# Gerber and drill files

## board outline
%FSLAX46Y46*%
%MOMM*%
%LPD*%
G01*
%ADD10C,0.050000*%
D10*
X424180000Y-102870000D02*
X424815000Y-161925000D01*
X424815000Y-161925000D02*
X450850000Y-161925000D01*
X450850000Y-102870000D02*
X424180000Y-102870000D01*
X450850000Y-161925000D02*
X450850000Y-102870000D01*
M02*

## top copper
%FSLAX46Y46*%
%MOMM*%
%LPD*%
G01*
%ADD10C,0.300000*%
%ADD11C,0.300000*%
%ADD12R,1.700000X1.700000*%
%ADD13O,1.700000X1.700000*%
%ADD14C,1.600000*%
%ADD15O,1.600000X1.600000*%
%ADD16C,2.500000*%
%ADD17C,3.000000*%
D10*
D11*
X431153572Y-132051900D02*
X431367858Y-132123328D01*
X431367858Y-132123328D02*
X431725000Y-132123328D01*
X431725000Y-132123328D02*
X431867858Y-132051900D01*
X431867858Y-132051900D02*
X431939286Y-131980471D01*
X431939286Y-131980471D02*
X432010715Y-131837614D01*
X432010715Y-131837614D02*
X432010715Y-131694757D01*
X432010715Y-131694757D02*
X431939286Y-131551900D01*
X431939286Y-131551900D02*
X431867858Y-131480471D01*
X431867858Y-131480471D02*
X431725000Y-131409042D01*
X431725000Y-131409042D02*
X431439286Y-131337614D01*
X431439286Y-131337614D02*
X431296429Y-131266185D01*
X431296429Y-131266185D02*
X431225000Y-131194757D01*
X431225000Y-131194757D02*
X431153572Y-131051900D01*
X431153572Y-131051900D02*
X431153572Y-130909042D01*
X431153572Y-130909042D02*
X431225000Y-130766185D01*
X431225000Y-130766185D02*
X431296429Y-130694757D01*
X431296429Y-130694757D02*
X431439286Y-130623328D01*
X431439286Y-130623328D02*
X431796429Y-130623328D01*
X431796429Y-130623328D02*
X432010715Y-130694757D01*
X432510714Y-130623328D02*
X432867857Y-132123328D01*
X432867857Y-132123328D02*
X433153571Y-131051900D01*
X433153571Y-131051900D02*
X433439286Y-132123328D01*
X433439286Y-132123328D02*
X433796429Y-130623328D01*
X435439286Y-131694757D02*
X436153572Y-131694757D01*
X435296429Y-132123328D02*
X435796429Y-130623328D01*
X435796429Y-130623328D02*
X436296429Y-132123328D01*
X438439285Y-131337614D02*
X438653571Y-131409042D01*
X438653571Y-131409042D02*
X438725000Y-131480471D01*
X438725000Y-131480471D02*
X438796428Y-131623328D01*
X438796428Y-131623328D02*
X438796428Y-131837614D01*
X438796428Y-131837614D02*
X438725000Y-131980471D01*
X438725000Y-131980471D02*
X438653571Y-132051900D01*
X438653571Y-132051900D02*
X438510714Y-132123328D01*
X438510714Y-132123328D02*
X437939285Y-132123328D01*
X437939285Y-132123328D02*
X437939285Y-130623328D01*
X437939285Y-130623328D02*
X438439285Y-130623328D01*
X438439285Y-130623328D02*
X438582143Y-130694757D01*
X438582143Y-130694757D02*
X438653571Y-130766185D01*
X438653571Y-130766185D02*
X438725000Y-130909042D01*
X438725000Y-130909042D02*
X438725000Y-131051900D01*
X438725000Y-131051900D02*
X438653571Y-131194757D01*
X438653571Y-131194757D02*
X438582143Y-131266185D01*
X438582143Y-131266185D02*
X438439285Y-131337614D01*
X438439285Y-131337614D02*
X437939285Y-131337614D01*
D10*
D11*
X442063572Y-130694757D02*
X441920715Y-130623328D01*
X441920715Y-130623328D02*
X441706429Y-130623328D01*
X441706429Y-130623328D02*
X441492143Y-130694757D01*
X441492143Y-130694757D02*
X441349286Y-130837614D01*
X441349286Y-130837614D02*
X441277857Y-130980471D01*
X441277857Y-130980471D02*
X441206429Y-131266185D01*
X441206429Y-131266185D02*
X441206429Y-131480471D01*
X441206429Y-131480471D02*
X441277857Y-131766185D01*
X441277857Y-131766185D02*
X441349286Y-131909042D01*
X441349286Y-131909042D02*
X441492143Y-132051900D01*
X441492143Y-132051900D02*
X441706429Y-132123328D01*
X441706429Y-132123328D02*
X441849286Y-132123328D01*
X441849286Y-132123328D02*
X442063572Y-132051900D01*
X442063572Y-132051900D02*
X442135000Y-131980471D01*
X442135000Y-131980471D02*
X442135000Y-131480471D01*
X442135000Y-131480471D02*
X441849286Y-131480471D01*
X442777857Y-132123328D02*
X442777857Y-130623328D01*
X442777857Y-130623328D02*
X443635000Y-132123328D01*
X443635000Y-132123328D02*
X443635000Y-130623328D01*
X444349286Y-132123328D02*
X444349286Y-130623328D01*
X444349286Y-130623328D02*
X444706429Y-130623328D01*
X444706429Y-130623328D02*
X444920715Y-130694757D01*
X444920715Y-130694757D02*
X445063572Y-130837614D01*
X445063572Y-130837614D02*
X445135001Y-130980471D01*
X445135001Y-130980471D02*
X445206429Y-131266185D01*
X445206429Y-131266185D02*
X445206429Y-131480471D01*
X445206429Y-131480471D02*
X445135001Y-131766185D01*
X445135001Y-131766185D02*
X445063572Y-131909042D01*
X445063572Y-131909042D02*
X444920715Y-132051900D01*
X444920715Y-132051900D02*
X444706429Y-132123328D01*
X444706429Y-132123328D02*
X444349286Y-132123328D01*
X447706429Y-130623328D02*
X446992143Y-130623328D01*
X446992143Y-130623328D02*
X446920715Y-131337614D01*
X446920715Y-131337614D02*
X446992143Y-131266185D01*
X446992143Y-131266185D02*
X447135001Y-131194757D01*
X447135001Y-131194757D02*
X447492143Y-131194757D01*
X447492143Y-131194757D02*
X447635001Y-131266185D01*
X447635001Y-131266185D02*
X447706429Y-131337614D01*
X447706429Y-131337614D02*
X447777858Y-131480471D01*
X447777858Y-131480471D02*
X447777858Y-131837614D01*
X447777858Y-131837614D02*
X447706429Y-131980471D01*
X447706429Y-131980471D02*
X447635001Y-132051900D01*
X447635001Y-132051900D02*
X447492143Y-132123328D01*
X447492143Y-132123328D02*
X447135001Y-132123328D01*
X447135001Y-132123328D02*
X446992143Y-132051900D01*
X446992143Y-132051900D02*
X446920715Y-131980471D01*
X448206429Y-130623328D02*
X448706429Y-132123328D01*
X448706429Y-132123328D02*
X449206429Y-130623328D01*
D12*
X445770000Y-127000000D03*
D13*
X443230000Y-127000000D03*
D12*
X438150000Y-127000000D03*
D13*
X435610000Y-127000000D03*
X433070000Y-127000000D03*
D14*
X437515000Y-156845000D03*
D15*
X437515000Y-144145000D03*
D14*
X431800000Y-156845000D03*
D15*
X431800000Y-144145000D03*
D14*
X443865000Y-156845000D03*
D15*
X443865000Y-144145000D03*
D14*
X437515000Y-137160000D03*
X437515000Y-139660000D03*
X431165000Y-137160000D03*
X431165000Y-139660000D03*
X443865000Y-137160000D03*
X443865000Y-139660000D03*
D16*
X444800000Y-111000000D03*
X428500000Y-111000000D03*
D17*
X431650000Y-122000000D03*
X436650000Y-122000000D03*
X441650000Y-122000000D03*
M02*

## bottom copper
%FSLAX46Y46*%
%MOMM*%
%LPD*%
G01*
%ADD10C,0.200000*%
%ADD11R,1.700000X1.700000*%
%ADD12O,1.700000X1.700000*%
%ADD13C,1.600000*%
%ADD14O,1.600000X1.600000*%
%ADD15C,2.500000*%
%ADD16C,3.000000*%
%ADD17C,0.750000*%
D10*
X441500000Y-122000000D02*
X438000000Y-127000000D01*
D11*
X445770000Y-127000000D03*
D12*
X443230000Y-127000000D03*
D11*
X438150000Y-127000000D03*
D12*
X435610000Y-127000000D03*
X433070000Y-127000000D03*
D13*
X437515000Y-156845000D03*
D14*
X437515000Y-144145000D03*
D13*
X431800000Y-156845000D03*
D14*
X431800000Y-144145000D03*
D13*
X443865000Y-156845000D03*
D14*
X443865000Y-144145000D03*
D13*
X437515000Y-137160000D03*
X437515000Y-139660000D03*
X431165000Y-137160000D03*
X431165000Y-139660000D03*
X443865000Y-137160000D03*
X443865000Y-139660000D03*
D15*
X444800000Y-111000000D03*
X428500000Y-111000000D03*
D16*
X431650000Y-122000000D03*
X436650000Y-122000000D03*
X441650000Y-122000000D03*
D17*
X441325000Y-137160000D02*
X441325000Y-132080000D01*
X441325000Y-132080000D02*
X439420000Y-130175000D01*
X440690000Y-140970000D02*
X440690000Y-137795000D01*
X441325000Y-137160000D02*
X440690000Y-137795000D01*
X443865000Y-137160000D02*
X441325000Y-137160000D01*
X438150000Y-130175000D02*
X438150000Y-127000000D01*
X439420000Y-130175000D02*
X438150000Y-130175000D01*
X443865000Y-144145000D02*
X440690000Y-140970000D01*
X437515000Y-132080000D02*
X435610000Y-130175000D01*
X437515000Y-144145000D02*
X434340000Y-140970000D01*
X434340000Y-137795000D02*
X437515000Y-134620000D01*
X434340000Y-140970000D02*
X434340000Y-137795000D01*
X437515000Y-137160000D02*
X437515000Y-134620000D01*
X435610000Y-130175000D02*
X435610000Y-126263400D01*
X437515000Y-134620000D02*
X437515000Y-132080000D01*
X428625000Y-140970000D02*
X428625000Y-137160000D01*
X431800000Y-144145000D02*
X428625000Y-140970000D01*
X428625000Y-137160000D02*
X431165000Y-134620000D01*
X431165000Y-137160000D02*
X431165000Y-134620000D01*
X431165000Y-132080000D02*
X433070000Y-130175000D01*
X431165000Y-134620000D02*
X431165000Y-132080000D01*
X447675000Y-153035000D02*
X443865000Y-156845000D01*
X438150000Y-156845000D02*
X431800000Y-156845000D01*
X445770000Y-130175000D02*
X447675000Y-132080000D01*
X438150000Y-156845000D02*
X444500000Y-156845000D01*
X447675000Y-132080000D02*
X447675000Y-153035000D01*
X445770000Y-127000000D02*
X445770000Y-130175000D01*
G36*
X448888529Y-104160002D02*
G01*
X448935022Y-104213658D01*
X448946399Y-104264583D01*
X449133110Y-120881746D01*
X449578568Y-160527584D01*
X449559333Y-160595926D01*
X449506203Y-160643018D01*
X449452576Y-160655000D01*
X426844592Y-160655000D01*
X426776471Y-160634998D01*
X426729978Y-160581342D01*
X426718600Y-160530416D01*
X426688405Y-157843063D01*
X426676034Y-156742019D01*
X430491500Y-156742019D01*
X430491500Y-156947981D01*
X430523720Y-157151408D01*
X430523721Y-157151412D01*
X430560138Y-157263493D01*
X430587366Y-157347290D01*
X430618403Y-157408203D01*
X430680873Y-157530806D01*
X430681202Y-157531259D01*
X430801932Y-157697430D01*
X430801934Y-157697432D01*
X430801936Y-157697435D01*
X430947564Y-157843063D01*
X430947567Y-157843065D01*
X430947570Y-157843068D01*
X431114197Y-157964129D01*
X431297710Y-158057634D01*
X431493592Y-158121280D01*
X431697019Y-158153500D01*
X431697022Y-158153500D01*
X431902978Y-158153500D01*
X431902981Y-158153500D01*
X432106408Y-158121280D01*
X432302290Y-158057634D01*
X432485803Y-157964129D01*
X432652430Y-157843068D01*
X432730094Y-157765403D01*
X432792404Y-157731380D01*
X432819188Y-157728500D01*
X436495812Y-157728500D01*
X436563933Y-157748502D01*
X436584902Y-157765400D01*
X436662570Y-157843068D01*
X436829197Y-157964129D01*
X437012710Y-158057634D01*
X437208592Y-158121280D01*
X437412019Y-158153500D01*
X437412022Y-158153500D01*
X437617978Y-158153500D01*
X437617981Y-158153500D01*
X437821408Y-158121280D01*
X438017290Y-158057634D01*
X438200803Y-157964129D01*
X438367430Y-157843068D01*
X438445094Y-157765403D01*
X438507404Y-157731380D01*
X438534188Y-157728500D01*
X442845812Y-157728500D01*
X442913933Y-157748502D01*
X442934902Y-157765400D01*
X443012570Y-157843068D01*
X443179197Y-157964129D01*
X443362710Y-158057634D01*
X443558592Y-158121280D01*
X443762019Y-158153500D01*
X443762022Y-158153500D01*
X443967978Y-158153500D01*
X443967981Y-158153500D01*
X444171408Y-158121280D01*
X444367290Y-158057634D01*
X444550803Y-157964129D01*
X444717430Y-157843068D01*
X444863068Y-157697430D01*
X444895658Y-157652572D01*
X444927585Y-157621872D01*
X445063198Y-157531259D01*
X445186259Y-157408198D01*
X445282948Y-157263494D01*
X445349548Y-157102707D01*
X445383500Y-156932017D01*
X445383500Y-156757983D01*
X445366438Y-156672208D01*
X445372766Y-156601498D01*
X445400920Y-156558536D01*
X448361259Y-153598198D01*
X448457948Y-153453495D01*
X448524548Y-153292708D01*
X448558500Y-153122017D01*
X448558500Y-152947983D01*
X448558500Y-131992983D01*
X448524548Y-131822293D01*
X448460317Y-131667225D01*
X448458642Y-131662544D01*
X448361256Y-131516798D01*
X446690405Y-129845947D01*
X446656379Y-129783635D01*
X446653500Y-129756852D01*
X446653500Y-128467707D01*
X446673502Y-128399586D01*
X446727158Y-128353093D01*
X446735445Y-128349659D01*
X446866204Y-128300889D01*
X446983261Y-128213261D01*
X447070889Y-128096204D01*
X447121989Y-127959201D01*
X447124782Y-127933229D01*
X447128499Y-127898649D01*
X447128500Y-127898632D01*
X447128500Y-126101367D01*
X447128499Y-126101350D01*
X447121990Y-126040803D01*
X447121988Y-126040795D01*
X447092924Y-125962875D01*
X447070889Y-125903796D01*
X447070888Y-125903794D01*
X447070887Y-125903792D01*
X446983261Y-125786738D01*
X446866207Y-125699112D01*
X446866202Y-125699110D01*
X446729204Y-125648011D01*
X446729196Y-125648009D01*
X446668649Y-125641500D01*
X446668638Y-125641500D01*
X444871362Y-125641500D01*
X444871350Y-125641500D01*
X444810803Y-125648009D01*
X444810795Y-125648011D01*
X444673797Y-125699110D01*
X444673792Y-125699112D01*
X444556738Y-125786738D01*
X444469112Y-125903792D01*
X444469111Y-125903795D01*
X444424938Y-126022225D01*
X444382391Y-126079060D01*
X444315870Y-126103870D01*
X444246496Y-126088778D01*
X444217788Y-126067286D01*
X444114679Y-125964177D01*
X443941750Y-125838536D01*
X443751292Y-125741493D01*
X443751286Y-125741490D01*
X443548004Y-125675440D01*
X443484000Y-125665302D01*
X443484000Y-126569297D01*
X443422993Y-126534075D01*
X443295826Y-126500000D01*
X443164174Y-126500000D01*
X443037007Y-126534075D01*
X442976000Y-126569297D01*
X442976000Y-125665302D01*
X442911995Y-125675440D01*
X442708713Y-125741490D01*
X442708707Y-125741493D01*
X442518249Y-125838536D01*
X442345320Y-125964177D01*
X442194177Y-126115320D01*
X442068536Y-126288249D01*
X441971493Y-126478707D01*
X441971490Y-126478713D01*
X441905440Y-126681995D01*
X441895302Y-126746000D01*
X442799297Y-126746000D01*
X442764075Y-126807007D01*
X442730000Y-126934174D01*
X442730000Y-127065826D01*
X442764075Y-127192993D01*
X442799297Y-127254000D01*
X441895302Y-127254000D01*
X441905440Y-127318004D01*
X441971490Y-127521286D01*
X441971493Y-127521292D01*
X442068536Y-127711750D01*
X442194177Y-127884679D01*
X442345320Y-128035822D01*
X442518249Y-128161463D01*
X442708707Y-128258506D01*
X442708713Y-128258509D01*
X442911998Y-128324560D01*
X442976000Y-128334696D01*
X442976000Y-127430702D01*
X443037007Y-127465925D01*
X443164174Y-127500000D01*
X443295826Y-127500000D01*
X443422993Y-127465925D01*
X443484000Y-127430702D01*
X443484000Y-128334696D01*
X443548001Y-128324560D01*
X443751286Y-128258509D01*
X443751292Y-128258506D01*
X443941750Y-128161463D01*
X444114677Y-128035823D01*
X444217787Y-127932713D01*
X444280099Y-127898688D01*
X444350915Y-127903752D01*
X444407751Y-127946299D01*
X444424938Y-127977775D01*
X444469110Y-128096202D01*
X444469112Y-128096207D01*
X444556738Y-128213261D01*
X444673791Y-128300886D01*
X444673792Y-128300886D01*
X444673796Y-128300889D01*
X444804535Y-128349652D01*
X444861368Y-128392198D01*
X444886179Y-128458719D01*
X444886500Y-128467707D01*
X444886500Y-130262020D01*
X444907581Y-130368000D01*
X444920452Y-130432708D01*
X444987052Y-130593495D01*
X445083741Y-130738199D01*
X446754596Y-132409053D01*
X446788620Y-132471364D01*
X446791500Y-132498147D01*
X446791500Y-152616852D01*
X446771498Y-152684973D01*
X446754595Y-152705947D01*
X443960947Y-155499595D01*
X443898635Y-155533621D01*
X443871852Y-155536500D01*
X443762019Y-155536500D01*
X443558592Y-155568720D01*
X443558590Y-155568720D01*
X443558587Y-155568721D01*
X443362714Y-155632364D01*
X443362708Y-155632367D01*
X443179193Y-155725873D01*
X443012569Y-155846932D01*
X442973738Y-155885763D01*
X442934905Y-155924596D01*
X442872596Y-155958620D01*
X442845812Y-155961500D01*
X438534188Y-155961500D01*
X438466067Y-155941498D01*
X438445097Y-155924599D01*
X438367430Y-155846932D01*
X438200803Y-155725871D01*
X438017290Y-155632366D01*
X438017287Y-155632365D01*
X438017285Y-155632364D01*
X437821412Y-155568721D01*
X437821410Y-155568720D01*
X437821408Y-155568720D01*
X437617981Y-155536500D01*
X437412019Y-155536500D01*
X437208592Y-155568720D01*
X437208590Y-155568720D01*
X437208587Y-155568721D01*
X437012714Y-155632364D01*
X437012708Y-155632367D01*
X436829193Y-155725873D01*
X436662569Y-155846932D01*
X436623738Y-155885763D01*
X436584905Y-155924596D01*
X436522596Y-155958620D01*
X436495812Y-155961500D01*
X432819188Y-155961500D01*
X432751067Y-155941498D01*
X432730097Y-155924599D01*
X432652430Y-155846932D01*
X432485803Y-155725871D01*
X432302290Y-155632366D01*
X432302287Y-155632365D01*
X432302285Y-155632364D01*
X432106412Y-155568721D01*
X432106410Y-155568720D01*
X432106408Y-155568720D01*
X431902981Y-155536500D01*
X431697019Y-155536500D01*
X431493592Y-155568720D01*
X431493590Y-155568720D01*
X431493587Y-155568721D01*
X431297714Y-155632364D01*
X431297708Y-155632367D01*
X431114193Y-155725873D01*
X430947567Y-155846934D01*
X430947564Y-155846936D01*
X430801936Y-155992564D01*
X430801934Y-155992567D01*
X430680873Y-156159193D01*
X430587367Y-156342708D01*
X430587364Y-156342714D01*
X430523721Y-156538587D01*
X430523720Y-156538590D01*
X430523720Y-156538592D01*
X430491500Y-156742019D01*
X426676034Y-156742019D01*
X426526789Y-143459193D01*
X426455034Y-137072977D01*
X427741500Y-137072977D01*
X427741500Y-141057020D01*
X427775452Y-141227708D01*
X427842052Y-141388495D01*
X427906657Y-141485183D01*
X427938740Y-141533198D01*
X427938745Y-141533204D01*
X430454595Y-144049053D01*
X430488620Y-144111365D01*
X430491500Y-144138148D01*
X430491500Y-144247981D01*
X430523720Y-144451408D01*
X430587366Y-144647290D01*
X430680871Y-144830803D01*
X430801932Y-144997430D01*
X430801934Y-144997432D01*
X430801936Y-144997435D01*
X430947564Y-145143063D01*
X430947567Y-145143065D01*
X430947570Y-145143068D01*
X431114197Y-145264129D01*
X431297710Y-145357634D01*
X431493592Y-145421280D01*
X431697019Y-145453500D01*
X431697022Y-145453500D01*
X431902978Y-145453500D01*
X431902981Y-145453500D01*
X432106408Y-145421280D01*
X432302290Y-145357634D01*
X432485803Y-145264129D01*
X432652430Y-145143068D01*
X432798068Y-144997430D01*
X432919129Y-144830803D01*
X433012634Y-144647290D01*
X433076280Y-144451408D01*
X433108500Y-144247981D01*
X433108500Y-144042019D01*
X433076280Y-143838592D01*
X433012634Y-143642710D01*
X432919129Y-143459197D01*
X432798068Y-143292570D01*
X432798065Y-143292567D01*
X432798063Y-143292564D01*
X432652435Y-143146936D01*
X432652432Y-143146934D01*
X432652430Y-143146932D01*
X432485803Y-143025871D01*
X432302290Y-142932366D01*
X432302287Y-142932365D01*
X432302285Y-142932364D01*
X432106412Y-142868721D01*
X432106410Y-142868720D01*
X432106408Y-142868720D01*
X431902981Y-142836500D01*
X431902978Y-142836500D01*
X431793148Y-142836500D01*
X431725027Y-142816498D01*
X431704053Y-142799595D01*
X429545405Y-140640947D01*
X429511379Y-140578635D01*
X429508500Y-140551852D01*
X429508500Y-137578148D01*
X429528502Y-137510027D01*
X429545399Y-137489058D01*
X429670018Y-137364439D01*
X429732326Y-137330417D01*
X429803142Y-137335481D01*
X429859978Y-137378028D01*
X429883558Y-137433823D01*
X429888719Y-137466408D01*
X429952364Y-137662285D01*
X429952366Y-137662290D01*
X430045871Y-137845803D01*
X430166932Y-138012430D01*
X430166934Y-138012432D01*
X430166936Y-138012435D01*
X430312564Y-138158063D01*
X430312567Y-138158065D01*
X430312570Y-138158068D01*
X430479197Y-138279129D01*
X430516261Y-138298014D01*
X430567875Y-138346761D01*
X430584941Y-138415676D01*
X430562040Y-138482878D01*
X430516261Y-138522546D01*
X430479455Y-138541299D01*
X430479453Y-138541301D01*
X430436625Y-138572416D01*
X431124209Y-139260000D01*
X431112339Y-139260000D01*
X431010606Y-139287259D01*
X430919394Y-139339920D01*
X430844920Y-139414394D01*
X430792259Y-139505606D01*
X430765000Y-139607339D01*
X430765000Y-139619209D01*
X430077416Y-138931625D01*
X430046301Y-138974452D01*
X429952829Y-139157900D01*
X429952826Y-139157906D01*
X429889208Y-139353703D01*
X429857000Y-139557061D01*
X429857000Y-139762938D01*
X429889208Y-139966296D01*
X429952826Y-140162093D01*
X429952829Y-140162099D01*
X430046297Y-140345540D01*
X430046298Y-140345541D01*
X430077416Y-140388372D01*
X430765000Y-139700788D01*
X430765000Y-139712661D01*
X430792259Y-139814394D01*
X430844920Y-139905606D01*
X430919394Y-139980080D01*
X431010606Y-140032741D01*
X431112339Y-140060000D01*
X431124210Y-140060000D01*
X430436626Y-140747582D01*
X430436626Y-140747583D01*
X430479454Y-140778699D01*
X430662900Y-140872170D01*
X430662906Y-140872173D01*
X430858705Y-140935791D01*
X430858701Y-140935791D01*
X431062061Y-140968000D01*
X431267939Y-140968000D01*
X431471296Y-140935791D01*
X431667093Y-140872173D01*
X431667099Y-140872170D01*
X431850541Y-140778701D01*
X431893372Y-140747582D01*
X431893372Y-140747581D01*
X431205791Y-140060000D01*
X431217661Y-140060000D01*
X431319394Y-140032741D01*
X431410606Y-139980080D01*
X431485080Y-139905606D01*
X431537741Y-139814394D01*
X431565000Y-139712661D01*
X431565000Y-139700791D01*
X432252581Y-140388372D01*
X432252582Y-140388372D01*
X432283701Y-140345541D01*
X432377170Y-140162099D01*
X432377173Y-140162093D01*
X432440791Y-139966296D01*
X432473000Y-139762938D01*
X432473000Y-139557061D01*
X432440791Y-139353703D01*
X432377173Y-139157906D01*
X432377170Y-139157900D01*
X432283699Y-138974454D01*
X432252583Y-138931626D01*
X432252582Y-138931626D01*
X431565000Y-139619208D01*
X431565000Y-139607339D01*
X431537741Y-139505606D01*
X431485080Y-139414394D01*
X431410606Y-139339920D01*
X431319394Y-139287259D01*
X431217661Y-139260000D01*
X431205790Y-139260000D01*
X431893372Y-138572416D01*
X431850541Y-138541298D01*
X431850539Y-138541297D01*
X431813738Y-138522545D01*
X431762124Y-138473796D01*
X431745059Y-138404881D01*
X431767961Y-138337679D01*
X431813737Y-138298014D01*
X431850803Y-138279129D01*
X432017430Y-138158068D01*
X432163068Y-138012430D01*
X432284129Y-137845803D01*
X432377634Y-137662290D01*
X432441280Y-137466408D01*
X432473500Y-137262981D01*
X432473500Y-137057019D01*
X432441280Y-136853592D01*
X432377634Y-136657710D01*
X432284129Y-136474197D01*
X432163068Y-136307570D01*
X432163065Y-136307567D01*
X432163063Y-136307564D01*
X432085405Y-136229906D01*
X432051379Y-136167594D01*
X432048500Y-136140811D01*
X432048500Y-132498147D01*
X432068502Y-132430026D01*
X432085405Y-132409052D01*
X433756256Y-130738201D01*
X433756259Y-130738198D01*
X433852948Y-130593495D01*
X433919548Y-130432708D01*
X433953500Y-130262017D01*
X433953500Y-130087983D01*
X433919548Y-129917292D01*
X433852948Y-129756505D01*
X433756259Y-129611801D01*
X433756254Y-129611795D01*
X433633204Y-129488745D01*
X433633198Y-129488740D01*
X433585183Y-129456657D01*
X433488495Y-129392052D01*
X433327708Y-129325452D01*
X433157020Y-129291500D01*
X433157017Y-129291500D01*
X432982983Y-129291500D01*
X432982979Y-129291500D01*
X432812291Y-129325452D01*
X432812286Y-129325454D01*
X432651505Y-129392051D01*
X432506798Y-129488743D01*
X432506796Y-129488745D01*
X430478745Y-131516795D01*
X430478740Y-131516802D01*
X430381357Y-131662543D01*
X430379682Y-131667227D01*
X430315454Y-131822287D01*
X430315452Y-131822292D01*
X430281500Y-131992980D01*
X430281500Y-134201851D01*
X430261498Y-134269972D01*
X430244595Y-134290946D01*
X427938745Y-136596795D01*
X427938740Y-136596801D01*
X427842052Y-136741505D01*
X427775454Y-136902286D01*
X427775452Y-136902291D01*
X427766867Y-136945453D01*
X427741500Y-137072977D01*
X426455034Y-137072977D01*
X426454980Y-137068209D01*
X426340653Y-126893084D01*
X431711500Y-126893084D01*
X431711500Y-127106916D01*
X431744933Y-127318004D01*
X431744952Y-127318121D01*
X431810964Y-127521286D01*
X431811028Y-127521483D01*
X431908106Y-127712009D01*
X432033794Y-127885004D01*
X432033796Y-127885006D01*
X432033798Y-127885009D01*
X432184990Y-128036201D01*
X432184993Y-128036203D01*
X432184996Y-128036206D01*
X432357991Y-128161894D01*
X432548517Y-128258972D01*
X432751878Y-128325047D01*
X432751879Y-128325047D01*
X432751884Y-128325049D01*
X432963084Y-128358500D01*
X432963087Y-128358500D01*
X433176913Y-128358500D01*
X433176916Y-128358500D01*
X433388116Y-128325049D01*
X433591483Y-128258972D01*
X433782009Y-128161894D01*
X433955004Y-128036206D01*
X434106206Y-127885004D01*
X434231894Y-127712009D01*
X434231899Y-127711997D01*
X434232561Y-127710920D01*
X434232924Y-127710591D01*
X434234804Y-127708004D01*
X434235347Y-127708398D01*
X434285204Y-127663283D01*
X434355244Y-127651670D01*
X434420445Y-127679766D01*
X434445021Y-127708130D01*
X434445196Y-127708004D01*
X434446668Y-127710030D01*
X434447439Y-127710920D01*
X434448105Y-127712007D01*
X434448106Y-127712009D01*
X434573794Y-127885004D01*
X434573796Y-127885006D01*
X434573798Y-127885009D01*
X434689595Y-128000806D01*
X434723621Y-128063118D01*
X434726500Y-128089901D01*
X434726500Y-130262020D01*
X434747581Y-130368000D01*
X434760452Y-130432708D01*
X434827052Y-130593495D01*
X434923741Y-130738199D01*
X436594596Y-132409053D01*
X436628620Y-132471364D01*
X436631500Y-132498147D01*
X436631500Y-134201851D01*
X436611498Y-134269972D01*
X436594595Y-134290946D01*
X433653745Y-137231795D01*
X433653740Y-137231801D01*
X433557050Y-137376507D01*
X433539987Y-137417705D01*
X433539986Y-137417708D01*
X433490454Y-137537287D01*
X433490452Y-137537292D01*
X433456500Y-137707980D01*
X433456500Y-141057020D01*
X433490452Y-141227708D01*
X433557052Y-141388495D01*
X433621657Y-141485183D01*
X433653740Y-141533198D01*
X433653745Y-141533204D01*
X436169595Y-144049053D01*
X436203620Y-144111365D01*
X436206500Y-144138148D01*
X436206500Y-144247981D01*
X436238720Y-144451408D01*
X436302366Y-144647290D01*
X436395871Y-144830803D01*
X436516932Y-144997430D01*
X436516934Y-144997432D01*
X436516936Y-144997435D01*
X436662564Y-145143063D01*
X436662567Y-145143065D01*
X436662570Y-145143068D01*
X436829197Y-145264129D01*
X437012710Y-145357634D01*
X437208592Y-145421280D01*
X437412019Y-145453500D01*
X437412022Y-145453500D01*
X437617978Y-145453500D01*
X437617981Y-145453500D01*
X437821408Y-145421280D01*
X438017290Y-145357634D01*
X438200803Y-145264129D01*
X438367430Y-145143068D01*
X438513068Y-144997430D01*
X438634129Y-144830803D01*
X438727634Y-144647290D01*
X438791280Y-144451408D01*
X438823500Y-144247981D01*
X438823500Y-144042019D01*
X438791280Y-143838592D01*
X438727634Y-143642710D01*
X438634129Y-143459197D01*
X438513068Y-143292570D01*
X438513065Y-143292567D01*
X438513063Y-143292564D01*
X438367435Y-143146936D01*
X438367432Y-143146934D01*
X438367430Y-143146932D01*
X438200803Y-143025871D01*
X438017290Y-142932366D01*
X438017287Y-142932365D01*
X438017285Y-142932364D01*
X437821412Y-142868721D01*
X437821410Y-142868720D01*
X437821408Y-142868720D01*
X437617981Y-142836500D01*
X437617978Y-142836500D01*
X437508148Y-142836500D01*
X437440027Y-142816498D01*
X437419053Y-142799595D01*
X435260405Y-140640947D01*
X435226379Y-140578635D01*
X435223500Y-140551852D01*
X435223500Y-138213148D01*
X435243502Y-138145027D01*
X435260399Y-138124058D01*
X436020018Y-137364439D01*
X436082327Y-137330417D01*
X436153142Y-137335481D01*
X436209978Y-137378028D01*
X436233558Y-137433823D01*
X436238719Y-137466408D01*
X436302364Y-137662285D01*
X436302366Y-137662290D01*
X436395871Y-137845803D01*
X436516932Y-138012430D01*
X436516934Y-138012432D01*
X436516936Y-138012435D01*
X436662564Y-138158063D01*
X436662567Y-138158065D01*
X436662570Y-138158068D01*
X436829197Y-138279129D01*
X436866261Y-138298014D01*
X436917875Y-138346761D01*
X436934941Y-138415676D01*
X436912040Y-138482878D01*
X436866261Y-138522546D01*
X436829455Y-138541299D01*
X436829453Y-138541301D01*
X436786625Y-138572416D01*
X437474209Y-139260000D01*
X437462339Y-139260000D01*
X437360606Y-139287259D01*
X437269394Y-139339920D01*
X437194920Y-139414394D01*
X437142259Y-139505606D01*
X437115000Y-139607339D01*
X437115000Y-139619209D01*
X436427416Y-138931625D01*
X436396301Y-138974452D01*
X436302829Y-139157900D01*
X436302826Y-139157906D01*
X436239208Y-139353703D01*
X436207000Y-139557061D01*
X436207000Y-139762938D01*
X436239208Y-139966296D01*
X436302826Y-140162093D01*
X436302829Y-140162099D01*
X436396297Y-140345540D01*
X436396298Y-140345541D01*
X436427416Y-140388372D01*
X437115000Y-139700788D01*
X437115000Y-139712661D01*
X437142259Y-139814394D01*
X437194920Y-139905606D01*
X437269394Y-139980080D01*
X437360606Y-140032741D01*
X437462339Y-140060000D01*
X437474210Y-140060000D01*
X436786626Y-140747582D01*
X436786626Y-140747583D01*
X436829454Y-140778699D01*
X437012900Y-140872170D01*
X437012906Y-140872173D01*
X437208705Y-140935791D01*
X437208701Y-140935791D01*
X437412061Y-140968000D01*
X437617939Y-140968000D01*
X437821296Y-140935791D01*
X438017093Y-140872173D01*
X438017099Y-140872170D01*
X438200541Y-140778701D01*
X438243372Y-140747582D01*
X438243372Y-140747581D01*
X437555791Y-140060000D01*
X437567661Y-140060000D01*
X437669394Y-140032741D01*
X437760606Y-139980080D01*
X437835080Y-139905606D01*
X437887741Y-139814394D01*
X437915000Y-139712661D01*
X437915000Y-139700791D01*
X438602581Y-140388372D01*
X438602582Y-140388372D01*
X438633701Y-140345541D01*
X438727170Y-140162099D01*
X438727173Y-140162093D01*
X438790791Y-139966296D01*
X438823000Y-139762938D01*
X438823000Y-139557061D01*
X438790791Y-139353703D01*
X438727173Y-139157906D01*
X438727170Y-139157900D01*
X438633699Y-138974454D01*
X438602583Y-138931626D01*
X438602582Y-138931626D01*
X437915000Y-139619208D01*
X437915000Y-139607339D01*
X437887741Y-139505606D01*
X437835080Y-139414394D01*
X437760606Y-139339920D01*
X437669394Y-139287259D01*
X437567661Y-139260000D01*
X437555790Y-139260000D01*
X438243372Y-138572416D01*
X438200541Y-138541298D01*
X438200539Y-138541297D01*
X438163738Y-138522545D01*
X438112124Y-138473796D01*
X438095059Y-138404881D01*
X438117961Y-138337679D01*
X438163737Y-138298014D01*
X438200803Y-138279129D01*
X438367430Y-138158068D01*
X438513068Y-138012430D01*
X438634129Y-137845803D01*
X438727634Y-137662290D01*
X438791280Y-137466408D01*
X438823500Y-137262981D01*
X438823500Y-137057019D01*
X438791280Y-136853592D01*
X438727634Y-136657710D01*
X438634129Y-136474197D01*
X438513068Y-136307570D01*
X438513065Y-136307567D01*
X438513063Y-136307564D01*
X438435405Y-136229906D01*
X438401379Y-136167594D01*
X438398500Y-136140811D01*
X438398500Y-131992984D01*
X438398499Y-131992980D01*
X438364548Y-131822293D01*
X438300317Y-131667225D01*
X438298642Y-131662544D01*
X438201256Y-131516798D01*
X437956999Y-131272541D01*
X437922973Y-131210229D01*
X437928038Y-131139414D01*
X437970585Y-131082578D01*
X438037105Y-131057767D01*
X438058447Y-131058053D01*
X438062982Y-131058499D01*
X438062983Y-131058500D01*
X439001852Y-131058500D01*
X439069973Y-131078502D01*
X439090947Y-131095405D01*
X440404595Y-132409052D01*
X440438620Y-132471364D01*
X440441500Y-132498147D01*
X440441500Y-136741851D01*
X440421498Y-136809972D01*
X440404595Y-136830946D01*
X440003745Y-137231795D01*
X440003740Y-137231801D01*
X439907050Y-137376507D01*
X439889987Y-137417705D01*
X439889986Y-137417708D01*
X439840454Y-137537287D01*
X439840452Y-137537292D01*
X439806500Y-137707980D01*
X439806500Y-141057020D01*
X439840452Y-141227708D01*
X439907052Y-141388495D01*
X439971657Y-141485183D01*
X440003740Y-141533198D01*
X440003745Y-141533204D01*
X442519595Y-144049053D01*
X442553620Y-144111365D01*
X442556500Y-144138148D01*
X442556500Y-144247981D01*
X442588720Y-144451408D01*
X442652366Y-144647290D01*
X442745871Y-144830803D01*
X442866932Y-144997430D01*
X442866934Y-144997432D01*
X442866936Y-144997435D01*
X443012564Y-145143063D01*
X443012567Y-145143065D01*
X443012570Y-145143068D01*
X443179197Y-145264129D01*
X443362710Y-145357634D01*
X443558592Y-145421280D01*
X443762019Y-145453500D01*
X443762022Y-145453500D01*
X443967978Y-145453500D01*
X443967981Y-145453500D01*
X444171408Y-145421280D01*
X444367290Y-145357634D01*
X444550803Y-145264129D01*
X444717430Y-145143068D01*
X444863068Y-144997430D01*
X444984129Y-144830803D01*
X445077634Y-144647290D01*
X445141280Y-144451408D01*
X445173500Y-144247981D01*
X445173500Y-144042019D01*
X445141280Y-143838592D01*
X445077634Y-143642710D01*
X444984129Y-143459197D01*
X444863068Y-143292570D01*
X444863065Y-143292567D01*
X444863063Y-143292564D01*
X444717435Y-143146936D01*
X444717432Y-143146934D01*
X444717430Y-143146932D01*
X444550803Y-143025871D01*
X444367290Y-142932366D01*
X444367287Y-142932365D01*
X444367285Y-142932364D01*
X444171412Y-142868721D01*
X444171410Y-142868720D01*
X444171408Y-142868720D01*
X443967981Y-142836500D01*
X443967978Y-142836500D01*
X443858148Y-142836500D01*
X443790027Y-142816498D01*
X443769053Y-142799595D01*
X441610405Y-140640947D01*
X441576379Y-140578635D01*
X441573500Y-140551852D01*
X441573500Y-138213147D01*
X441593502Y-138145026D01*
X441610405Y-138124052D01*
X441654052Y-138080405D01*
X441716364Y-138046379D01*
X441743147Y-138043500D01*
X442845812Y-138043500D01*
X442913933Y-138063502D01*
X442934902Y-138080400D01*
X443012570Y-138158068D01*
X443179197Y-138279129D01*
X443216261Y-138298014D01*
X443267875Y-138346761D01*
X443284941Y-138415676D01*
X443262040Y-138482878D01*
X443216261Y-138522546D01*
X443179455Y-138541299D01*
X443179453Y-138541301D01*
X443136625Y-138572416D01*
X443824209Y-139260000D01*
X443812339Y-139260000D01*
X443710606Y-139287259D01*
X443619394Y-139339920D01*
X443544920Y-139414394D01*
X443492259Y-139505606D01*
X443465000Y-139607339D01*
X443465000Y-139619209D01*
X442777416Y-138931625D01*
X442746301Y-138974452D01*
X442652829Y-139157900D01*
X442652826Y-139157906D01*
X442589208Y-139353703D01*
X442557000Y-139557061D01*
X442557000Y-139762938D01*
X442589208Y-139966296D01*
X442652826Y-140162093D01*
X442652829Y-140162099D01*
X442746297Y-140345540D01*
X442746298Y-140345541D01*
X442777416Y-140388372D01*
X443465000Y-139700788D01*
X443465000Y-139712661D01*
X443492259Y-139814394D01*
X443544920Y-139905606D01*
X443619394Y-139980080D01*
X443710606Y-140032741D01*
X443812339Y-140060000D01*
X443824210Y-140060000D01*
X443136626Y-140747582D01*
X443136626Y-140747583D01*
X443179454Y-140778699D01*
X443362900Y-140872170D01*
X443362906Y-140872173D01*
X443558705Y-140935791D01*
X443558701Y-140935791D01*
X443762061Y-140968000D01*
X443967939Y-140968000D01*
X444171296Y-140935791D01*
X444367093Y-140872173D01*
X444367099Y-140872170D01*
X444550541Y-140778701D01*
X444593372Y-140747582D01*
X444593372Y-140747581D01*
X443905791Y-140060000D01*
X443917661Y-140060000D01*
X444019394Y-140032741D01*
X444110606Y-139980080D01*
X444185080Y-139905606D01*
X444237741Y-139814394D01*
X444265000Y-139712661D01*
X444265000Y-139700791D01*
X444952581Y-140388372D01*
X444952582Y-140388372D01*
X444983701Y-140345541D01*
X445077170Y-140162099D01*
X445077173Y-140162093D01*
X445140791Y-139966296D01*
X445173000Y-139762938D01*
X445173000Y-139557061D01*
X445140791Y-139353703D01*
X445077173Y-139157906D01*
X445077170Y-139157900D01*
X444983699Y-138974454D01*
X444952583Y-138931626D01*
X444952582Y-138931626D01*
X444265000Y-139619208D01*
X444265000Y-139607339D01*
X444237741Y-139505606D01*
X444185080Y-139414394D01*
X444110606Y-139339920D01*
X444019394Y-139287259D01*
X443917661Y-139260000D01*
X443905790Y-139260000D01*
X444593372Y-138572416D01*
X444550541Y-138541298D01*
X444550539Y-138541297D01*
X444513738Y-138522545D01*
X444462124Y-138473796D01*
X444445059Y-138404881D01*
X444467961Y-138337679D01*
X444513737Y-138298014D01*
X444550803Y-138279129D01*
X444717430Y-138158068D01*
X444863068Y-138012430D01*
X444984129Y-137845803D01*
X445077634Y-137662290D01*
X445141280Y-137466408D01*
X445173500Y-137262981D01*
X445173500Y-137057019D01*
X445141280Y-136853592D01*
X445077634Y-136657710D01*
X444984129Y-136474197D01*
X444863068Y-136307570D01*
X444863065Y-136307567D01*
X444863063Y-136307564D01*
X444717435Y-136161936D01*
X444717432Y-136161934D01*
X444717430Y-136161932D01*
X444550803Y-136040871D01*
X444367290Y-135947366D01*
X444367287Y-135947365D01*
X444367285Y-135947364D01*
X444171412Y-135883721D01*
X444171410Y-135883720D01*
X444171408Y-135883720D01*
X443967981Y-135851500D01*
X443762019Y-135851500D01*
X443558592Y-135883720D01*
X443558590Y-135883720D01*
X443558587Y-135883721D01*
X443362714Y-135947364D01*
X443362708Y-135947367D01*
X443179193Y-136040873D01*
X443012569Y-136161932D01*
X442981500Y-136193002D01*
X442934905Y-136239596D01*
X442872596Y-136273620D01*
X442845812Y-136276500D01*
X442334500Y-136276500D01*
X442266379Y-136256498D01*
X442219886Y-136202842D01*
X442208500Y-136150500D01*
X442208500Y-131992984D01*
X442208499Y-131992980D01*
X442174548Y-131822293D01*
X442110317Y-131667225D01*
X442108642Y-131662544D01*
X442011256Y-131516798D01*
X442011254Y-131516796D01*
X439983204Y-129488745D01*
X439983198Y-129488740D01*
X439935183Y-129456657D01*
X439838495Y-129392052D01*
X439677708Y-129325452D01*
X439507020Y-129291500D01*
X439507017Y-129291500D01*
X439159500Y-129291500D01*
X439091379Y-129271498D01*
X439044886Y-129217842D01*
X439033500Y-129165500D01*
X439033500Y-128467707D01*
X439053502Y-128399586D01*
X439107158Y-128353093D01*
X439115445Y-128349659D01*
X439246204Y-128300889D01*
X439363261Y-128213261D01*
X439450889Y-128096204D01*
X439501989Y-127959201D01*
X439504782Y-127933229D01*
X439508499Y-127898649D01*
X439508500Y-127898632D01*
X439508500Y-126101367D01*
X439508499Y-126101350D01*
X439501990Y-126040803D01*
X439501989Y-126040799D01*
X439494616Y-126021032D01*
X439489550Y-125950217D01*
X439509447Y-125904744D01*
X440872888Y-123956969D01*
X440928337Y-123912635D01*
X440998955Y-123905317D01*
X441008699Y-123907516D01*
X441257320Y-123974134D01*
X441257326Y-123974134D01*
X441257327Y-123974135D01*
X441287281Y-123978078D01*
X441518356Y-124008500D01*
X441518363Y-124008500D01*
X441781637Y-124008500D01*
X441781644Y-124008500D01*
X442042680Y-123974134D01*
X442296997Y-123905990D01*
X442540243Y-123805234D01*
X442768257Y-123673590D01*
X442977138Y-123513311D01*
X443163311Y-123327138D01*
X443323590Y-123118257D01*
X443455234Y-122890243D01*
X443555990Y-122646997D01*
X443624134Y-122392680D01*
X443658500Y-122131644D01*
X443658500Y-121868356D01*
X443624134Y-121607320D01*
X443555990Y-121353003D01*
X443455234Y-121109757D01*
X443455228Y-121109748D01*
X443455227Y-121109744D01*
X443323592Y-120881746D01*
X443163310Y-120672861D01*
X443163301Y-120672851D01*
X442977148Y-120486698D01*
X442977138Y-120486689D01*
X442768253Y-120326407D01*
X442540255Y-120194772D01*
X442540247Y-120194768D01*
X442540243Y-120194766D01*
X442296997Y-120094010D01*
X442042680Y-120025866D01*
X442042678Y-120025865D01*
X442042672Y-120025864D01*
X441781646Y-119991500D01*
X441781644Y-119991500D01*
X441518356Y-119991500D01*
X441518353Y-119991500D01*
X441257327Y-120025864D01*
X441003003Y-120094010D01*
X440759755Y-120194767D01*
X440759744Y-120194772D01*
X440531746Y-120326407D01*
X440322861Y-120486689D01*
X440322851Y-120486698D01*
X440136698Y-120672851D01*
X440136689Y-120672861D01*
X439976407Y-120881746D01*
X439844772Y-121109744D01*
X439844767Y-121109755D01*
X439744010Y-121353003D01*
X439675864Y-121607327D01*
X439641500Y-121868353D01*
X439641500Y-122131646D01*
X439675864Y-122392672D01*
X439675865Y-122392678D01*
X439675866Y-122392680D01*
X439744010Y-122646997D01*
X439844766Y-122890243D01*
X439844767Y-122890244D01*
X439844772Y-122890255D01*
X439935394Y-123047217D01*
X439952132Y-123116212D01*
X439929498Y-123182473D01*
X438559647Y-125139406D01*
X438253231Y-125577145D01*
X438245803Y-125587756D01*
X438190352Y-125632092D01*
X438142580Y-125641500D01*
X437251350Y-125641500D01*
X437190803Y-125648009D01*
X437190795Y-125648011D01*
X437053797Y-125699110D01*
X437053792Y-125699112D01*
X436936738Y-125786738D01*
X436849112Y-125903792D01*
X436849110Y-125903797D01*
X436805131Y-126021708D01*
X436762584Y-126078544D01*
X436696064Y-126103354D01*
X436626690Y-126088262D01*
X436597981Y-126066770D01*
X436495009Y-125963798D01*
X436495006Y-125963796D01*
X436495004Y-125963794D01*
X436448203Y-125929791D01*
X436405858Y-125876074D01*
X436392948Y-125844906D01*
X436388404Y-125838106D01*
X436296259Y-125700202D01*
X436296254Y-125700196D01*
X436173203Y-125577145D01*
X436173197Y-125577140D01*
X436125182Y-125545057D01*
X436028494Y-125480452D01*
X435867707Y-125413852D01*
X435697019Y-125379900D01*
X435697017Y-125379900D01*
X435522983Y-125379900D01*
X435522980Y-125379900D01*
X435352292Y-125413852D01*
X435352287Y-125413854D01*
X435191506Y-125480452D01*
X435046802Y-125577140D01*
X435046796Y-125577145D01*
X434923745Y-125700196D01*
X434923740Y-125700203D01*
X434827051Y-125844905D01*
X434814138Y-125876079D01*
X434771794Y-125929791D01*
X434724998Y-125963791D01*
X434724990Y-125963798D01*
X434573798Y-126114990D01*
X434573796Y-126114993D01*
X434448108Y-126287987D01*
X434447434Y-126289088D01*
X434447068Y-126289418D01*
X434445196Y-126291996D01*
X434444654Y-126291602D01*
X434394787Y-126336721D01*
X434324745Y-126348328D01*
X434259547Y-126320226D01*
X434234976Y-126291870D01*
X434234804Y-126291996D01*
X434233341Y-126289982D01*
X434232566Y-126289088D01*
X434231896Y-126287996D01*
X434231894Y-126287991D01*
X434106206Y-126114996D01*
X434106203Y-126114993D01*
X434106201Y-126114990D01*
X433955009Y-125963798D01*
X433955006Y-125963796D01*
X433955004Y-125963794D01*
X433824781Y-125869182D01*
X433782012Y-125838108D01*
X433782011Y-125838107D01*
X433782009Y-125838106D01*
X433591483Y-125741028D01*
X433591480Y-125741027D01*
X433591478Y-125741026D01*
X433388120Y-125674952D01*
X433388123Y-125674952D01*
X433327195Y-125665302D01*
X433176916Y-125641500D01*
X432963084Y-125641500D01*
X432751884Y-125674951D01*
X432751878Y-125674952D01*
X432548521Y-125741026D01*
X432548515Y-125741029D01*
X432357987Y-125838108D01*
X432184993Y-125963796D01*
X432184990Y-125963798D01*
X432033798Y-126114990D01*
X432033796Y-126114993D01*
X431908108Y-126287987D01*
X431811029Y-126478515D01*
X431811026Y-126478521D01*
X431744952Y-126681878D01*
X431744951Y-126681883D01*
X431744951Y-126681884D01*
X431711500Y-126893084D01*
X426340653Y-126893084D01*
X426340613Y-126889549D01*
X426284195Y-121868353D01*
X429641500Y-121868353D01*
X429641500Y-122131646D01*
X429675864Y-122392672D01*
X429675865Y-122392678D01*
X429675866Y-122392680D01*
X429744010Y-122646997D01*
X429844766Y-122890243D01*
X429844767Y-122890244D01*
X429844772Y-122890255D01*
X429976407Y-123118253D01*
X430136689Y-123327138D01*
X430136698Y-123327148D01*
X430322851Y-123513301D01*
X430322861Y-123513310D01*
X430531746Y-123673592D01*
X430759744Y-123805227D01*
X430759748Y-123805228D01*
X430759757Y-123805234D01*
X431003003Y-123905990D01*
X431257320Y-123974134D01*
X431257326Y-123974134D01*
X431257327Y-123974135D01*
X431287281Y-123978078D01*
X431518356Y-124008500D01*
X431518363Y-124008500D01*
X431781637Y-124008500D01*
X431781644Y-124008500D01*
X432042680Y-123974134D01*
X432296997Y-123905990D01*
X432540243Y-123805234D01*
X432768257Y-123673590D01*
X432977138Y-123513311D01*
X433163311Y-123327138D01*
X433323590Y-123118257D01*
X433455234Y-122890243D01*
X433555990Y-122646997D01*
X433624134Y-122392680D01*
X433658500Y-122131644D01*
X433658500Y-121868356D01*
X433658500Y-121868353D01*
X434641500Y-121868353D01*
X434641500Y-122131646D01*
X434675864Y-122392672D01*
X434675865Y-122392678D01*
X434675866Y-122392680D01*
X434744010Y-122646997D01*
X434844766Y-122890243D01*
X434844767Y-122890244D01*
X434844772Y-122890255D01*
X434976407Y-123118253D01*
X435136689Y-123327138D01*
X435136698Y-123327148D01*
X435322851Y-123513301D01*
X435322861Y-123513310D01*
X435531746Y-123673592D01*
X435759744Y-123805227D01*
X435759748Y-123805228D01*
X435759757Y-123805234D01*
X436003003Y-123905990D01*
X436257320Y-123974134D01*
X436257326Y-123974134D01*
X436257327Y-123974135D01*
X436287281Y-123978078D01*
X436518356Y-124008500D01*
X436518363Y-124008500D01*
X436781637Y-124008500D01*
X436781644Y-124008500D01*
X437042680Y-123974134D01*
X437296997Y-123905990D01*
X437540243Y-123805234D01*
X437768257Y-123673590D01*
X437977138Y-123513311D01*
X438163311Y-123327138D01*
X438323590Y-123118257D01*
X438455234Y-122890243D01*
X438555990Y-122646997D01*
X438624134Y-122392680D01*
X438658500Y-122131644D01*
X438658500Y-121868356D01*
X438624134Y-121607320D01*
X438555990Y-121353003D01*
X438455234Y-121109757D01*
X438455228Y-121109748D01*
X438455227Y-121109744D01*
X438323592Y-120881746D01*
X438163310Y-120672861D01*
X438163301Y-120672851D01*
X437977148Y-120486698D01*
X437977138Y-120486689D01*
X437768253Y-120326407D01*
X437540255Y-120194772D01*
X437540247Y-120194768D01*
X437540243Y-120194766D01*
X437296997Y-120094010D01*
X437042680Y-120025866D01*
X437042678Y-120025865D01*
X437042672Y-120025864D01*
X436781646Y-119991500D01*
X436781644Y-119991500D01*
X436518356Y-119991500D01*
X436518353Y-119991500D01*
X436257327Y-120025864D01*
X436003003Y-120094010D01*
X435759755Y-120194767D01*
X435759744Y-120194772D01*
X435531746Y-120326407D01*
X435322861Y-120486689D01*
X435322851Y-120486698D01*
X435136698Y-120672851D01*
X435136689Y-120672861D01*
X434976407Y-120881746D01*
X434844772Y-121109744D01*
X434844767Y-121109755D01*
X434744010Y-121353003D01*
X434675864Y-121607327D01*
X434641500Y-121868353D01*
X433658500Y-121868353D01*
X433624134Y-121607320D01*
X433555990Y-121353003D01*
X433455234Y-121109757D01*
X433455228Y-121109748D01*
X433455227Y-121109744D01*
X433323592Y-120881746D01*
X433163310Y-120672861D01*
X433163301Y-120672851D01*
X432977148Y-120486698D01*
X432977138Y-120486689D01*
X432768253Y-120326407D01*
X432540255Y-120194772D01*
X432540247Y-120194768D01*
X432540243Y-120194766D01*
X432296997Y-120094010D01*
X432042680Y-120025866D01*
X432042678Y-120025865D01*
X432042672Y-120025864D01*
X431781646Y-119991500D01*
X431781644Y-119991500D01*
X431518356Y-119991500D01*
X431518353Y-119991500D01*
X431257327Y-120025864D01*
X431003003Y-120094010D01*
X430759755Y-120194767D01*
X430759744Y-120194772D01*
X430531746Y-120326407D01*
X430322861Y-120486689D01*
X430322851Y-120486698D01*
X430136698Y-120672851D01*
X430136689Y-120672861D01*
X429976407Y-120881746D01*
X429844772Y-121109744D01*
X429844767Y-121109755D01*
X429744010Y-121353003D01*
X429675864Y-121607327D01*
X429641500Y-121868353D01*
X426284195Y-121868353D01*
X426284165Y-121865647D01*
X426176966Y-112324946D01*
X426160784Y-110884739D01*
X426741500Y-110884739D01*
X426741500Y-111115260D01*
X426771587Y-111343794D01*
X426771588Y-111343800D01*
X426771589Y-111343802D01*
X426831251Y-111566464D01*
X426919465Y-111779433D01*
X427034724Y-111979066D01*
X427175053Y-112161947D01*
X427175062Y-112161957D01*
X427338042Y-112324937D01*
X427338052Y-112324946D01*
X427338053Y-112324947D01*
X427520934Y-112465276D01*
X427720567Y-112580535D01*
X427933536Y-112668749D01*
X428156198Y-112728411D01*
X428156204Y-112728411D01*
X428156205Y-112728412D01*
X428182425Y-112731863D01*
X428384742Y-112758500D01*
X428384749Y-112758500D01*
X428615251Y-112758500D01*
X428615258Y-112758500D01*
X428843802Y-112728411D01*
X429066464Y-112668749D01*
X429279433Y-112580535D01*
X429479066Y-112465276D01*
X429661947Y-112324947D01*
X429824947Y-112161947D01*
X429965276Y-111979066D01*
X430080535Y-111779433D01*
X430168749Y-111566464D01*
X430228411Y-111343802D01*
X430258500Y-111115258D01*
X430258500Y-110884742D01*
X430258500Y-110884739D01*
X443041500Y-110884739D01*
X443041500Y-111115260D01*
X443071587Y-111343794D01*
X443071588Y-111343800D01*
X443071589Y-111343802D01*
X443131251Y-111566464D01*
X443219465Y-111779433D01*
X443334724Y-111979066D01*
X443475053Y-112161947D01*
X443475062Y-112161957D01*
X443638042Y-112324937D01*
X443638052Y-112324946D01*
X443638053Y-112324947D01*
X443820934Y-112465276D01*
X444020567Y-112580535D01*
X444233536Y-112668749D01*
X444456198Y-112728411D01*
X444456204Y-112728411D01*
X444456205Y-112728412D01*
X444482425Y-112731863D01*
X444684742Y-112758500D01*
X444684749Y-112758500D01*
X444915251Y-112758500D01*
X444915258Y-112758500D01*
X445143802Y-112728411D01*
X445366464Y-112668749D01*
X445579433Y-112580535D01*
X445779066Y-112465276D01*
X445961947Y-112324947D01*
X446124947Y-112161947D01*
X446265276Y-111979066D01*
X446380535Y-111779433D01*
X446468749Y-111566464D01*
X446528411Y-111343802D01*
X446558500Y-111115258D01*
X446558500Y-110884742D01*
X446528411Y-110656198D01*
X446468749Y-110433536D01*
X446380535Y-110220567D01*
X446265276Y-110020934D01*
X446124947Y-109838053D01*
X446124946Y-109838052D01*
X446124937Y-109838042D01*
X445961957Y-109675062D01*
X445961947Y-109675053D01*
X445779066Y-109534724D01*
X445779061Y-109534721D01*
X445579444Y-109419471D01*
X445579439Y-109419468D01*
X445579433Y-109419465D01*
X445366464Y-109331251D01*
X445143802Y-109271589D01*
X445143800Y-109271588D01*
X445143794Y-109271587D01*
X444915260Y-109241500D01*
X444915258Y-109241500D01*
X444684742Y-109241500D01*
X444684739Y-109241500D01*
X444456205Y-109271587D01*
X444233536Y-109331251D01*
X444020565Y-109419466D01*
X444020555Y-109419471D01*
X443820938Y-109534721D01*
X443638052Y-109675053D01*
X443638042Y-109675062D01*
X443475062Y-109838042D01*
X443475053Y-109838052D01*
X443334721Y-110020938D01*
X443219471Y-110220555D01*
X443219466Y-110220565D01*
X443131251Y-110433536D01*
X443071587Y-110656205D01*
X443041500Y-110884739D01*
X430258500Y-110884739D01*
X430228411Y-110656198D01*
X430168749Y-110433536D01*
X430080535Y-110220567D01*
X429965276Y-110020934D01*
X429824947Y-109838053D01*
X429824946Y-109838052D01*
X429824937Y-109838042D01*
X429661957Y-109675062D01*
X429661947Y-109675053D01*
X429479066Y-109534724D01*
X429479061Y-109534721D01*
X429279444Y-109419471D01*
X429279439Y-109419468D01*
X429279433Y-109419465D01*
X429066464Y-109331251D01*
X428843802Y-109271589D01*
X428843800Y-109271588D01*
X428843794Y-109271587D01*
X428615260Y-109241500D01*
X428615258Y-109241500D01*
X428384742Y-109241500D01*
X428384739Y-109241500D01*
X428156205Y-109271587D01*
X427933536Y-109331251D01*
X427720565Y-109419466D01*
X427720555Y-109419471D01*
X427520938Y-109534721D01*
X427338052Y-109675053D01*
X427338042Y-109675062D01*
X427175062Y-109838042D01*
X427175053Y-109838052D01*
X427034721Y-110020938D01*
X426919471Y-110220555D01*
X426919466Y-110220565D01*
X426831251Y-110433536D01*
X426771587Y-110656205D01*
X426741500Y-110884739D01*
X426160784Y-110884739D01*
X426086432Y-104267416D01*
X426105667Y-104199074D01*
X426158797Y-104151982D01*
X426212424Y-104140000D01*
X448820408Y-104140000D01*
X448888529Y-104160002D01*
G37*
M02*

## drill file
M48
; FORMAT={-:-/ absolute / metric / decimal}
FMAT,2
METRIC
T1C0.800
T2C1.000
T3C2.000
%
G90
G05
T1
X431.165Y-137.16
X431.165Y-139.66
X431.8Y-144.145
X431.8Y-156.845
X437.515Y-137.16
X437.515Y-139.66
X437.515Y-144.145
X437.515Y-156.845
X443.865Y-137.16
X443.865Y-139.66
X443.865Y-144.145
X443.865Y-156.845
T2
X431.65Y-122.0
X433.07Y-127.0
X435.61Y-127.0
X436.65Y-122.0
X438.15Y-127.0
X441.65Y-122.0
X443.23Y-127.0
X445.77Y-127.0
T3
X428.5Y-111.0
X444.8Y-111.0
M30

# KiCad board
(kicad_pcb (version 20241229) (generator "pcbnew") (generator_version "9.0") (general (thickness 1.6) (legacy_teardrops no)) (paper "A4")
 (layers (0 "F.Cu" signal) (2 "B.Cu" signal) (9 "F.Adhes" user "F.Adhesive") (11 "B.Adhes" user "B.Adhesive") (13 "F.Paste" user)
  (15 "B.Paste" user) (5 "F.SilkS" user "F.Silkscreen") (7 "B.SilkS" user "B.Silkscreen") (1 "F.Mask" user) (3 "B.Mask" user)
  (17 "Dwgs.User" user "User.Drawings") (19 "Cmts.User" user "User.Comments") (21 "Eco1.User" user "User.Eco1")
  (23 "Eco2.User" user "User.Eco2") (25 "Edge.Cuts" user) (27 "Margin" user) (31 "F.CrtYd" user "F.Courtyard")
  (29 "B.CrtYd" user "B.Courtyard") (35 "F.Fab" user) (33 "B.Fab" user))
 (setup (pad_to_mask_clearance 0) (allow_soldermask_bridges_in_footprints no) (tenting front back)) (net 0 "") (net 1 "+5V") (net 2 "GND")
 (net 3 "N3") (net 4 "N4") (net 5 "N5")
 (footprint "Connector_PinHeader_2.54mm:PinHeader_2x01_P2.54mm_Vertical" (layer "F.Cu") (at 445.77 127 180)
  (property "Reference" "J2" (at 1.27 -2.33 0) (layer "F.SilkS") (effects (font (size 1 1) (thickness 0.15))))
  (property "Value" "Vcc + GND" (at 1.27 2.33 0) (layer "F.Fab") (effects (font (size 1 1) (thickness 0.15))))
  (pad "1" thru_hole rect (at 0 0 180) (size 1.7 1.7) (drill 1) (layers "*.Cu" "*.Mask") (remove_unused_layers no) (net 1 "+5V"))
  (pad "2" thru_hole oval (at 2.54 0 180) (size 1.7 1.7) (drill 1) (layers "*.Cu" "*.Mask") (remove_unused_layers no) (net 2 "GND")))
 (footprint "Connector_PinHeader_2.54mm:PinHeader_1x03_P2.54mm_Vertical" (layer "F.Cu") (at 438.15 127 -90)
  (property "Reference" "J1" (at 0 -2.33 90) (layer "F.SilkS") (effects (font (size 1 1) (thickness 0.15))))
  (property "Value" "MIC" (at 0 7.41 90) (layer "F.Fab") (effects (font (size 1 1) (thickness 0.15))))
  (pad "1" thru_hole rect (at 0 0 270) (size 1.7 1.7) (drill 1) (layers "*.Cu" "*.Mask") (remove_unused_layers no) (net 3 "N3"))
  (pad "2" thru_hole oval (at 0 2.54 270) (size 1.7 1.7) (drill 1) (layers "*.Cu" "*.Mask") (remove_unused_layers no) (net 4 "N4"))
  (pad "3" thru_hole oval (at 0 5.08 270) (size 1.7 1.7) (drill 1) (layers "*.Cu" "*.Mask") (remove_unused_layers no) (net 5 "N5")))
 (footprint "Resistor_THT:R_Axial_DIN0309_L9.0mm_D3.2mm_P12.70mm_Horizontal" (layer "F.Cu") (at 437.515 156.845 90)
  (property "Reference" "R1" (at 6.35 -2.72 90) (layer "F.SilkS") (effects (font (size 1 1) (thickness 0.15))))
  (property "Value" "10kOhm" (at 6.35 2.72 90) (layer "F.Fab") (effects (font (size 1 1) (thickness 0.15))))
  (pad "1" thru_hole circle (at 0 0 90) (size 1.6 1.6) (drill 0.8) (layers "*.Cu" "*.Mask") (remove_unused_layers no) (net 1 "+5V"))
  (pad "2" thru_hole oval (at 12.7 0 90) (size 1.6 1.6) (drill 0.8) (layers "*.Cu" "*.Mask") (remove_unused_layers no) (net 4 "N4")))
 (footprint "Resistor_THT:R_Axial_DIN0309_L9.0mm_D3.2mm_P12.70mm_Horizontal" (layer "F.Cu") (at 431.8 156.845 90)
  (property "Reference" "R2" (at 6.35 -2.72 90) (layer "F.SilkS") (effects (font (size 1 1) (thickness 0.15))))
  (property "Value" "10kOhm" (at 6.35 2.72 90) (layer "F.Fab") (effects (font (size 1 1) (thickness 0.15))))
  (pad "1" thru_hole circle (at 0 0 90) (size 1.6 1.6) (drill 0.8) (layers "*.Cu" "*.Mask") (remove_unused_layers no) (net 1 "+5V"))
  (pad "2" thru_hole oval (at 12.7 0 90) (size 1.6 1.6) (drill 0.8) (layers "*.Cu" "*.Mask") (remove_unused_layers no) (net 5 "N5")))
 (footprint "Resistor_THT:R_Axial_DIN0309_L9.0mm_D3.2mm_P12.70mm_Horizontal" (layer "F.Cu") (at 443.865 156.845 90)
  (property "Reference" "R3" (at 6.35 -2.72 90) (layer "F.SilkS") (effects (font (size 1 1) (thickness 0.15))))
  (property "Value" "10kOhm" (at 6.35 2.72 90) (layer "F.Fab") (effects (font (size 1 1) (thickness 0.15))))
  (pad "1" thru_hole circle (at 0 0 90) (size 1.6 1.6) (drill 0.8) (layers "*.Cu" "*.Mask") (remove_unused_layers no) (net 1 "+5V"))
  (pad "2" thru_hole oval (at 12.7 0 90) (size 1.6 1.6) (drill 0.8) (layers "*.Cu" "*.Mask") (remove_unused_layers no) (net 3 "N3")))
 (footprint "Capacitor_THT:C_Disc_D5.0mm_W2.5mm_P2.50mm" (layer "F.Cu") (at 437.515 137.16 -90)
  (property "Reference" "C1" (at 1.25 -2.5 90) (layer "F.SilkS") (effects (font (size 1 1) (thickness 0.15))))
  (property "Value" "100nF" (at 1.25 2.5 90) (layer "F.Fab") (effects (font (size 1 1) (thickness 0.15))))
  (pad "1" thru_hole circle (at 0 0 270) (size 1.6 1.6) (drill 0.8) (layers "*.Cu" "*.Mask") (remove_unused_layers no) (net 4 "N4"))
  (pad "2" thru_hole circle (at 2.5 0 270) (size 1.6 1.6) (drill 0.8) (layers "*.Cu" "*.Mask") (remove_unused_layers no) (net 2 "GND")))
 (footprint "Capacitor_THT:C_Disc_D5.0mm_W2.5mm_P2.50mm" (layer "F.Cu") (at 431.165 137.16 -90)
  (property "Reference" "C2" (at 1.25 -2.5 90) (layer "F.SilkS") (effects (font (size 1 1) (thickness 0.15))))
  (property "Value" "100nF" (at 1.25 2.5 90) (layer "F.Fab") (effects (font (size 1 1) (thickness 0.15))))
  (pad "1" thru_hole circle (at 0 0 270) (size 1.6 1.6) (drill 0.8) (layers "*.Cu" "*.Mask") (remove_unused_layers no) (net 5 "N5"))
  (pad "2" thru_hole circle (at 2.5 0 270) (size 1.6 1.6) (drill 0.8) (layers "*.Cu" "*.Mask") (remove_unused_layers no) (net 2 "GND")))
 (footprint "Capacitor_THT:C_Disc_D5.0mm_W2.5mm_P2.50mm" (layer "F.Cu") (at 443.865 137.16 -90)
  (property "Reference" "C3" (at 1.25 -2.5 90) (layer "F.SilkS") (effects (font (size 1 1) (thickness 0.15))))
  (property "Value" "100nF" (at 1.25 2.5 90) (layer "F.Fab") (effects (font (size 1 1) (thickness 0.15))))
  (pad "1" thru_hole circle (at 0 0 270) (size 1.6 1.6) (drill 0.8) (layers "*.Cu" "*.Mask") (remove_unused_layers no) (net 3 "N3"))
  (pad "2" thru_hole circle (at 2.5 0 270) (size 1.6 1.6) (drill 0.8) (layers "*.Cu" "*.Mask") (remove_unused_layers no) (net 2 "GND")))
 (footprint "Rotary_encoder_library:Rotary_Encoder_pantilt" (layer "F.Cu") (at 444.8 103 180)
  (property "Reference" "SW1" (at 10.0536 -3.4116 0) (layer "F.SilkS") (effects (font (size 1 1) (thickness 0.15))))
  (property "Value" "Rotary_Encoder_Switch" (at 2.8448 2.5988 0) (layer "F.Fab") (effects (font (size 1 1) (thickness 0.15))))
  (pad "1" thru_hole circle (at 0 -8 180) (size 2.5 2.5) (drill 2) (layers "*.Cu" "*.Mask") (remove_unused_layers no))
  (pad "2" thru_hole circle (at 16.3 -8 180) (size 2.5 2.5) (drill 2) (layers "*.Cu" "*.Mask") (remove_unused_layers no))
  (pad "A" thru_hole circle (at 13.15 -19 180) (size 3 3) (drill 1) (layers "*.Cu" "*.Mask") (remove_unused_layers no) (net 4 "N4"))
  (pad "B" thru_hole circle (at 8.15 -19 180) (size 3 3) (drill 1) (layers "*.Cu" "*.Mask") (remove_unused_layers no) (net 5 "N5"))
  (pad "C" thru_hole circle (at 3.15 -19 180) (size 3 3) (drill 1) (layers "*.Cu" "*.Mask") (remove_unused_layers no) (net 3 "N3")))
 (gr_line (start 441.5 122) (end 438 127) (stroke (width 0.2) (type default)) (layer "B.Cu") (net 3))
 (gr_line (start 424.18 102.87) (end 424.815 161.925) (stroke (width 0.05) (type solid)) (layer "Edge.Cuts"))
 (gr_line (start 424.815 161.925) (end 450.85 161.925) (stroke (width 0.05) (type solid)) (layer "Edge.Cuts"))
 (gr_line (start 450.85 102.87) (end 424.18 102.87) (stroke (width 0.05) (type solid)) (layer "Edge.Cuts"))
 (gr_line (start 450.85 161.925) (end 450.85 102.87) (stroke (width 0.05) (type solid)) (layer "Edge.Cuts"))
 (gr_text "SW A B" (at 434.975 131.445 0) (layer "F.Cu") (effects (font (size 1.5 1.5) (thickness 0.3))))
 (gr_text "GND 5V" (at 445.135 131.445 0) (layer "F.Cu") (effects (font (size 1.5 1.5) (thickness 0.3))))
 (segment (start 441.325 137.16) (end 441.325 132.08) (width 0.75) (layer "B.Cu") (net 3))
 (segment (start 441.325 132.08) (end 439.42 130.175) (width 0.75) (layer "B.Cu") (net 3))
 (segment (start 440.69 140.97) (end 440.69 137.795) (width 0.75) (layer "B.Cu") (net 3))
 (segment (start 441.325 137.16) (end 440.69 137.795) (width 0.75) (layer "B.Cu") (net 3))
 (segment (start 443.865 137.16) (end 441.325 137.16) (width 0.75) (layer "B.Cu") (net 3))
 (segment (start 438.15 130.175) (end 438.15 127) (width 0.75) (layer "B.Cu") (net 3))
 (segment (start 439.42 130.175) (end 438.15 130.175) (width 0.75) (layer "B.Cu") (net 3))
 (segment (start 443.865 144.145) (end 440.69 140.97) (width 0.75) (layer "B.Cu") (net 3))
 (segment (start 437.515 132.08) (end 435.61 130.175) (width 0.75) (layer "B.Cu") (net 4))
 (segment (start 437.515 144.145) (end 434.34 140.97) (width 0.75) (layer "B.Cu") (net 4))
 (segment (start 434.34 137.795) (end 437.515 134.62) (width 0.75) (layer "B.Cu") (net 4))
 (segment (start 434.34 140.97) (end 434.34 137.795) (width 0.75) (layer "B.Cu") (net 4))
 (segment (start 437.515 137.16) (end 437.515 134.62) (width 0.75) (layer "B.Cu") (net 4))
 (segment (start 435.61 130.175) (end 435.61 126.2634) (width 0.75) (layer "B.Cu") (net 4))
 (segment (start 437.515 134.62) (end 437.515 132.08) (width 0.75) (layer "B.Cu") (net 4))
 (segment (start 428.625 140.97) (end 428.625 137.16) (width 0.75) (layer "B.Cu") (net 5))
 (segment (start 431.8 144.145) (end 428.625 140.97) (width 0.75) (layer "B.Cu") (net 5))
 (segment (start 428.625 137.16) (end 431.165 134.62) (width 0.75) (layer "B.Cu") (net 5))
 (segment (start 431.165 137.16) (end 431.165 134.62) (width 0.75) (layer "B.Cu") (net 5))
 (segment (start 431.165 132.08) (end 433.07 130.175) (width 0.75) (layer "B.Cu") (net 5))
 (segment (start 431.165 134.62) (end 431.165 132.08) (width 0.75) (layer "B.Cu") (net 5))
 (segment (start 447.675 153.035) (end 443.865 156.845) (width 0.75) (layer "B.Cu") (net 1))
 (segment (start 438.15 156.845) (end 431.8 156.845) (width 0.75) (layer "B.Cu") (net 1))
 (segment (start 445.77 130.175) (end 447.675 132.08) (width 0.75) (layer "B.Cu") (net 1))
 (segment (start 438.15 156.845) (end 444.5 156.845) (width 0.75) (layer "B.Cu") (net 1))
 (segment (start 447.675 132.08) (end 447.675 153.035) (width 0.75) (layer "B.Cu") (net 1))
 (segment (start 445.77 127) (end 445.77 130.175) (width 0.75) (layer "B.Cu") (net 1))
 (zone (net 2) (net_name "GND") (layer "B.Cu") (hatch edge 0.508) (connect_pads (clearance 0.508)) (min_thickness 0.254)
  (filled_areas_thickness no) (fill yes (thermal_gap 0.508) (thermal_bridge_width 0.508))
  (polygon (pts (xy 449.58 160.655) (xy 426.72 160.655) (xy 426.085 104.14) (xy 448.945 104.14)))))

